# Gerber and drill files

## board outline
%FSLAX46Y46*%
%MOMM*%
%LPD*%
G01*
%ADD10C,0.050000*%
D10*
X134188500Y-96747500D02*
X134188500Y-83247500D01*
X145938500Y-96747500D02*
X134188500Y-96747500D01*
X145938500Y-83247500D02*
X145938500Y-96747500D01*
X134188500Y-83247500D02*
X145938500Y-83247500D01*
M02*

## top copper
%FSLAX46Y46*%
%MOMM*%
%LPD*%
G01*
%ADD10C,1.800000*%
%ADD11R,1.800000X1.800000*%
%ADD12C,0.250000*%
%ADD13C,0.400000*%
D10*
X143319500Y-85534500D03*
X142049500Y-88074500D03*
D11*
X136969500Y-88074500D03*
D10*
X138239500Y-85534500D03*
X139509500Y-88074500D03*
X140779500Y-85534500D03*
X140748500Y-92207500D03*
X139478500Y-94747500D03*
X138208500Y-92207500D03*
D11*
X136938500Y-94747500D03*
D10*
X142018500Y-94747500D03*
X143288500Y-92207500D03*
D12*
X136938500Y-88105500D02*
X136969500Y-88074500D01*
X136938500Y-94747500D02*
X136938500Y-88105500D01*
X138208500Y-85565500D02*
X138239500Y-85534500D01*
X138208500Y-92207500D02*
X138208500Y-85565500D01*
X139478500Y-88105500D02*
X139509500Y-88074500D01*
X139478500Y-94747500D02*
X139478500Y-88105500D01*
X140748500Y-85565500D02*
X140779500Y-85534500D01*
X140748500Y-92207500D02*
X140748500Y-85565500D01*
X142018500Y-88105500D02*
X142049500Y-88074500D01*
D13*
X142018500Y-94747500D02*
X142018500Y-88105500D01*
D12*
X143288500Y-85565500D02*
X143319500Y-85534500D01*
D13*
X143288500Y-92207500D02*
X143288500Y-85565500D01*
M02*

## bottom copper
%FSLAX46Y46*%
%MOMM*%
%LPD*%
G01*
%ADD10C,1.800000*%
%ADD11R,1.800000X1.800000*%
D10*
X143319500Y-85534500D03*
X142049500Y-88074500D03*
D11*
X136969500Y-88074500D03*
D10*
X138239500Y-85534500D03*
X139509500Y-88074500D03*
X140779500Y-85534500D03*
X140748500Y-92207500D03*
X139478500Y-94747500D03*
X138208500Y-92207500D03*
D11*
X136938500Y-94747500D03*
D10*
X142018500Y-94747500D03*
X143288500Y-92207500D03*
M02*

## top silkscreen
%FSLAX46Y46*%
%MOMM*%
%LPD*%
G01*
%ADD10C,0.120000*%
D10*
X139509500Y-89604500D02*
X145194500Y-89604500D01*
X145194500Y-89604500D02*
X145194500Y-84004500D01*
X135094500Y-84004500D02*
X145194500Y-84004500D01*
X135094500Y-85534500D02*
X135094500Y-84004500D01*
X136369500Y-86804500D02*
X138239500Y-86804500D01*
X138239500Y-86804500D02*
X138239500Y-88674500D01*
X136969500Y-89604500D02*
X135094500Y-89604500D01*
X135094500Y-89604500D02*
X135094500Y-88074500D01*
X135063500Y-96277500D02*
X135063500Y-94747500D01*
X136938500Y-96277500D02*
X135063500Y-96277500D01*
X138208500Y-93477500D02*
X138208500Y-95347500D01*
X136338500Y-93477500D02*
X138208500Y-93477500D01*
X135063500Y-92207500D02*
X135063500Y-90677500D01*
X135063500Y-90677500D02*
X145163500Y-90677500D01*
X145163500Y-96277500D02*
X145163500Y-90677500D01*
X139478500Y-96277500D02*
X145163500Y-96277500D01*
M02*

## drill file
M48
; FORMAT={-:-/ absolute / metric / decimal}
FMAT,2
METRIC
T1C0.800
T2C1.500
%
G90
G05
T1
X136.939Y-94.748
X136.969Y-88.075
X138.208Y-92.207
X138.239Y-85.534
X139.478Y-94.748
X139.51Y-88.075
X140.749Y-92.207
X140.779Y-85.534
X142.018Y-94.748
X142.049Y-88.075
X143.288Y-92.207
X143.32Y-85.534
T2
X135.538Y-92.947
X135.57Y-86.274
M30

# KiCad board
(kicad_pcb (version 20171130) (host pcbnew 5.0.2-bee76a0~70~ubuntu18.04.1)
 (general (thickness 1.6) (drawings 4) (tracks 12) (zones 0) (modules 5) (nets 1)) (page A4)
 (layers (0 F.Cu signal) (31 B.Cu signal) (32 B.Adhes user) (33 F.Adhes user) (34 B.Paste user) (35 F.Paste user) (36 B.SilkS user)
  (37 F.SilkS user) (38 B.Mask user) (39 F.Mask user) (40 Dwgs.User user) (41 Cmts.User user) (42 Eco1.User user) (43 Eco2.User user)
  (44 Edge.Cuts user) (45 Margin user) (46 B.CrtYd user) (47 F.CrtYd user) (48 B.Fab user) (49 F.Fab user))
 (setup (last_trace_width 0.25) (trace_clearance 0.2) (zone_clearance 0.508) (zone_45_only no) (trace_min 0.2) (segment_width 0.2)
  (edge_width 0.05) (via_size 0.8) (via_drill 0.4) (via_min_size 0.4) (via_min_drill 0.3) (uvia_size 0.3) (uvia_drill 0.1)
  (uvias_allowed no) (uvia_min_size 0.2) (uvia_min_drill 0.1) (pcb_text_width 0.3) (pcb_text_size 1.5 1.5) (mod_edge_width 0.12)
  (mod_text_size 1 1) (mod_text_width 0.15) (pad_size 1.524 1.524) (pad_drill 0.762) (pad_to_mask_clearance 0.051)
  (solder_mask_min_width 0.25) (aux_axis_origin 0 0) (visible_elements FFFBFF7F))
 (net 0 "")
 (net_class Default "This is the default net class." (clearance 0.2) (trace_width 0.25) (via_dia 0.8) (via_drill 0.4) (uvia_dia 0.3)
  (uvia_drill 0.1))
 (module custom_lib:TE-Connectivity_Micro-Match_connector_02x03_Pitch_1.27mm (layer F.Cu) (at 136.9695 88.0745 90)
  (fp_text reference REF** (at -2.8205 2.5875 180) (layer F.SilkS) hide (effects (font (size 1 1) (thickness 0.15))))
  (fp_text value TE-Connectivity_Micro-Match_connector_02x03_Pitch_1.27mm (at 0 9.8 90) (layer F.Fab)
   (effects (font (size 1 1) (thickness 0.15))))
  (fp_line (start -1.53 2.54) (end -1.53 8.225) (layer F.SilkS) (width 0.12))
  (fp_line (start -1.53 8.225) (end 4.07 8.225) (layer F.SilkS) (width 0.12))
  (fp_line (start 4.07 -1.875) (end 4.07 8.225) (layer F.SilkS) (width 0.12))
  (fp_line (start 2.54 -1.875) (end 4.07 -1.875) (layer F.SilkS) (width 0.12))
  (fp_line (start 1.27 -0.6) (end 1.27 1.27) (layer F.SilkS) (width 0.12))
  (fp_line (start 1.27 1.27) (end -0.6 1.27) (layer F.SilkS) (width 0.12))
  (fp_line (start -1.53 0) (end -1.53 -1.875) (layer F.SilkS) (width 0.12))
  (fp_line (start -1.53 -1.875) (end 0 -1.875) (layer F.SilkS) (width 0.12))
  (pad 6 thru_hole circle (at 2.54 6.35 90) (size 1.8 1.8) (drill 0.8001) (layers *.Cu *.Mask))
  (pad 5 thru_hole circle (at 0 5.08 90) (size 1.8 1.8) (drill 0.8001) (layers *.Cu *.Mask))
  (pad 1 thru_hole rect (at 0 0 90) (size 1.8 1.8) (drill 0.8001) (layers *.Cu *.Mask))
  (pad 2 thru_hole circle (at 2.54 1.27 90) (size 1.8 1.8) (drill 0.8001) (layers *.Cu *.Mask))
  (pad 3 thru_hole circle (at 0 2.54 90) (size 1.8 1.8) (drill 0.8001) (layers *.Cu *.Mask))
  (pad 4 thru_hole circle (at 2.54 3.81 90) (size 1.8 1.8) (drill 0.8001) (layers *.Cu *.Mask))
  (pad "" np_thru_hole circle (at 1.8 -1.4 90) (size 1.5001 1.5001) (drill 1.5001) (layers *.Cu *.Mask)))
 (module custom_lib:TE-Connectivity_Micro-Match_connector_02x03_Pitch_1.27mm (layer F.Cu) (at 136.9385 94.7475 90)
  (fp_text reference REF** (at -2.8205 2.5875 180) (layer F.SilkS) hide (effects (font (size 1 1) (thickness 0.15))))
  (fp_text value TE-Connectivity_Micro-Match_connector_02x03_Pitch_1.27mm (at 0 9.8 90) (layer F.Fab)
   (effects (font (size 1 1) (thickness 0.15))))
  (fp_line (start -1.53 -1.875) (end 0 -1.875) (layer F.SilkS) (width 0.12))
  (fp_line (start -1.53 0) (end -1.53 -1.875) (layer F.SilkS) (width 0.12))
  (fp_line (start 1.27 1.27) (end -0.6 1.27) (layer F.SilkS) (width 0.12))
  (fp_line (start 1.27 -0.6) (end 1.27 1.27) (layer F.SilkS) (width 0.12))
  (fp_line (start 2.54 -1.875) (end 4.07 -1.875) (layer F.SilkS) (width 0.12))
  (fp_line (start 4.07 -1.875) (end 4.07 8.225) (layer F.SilkS) (width 0.12))
  (fp_line (start -1.53 8.225) (end 4.07 8.225) (layer F.SilkS) (width 0.12))
  (fp_line (start -1.53 2.54) (end -1.53 8.225) (layer F.SilkS) (width 0.12))
  (pad "" np_thru_hole circle (at 1.8 -1.4 90) (size 1.5001 1.5001) (drill 1.5001) (layers *.Cu *.Mask))
  (pad 4 thru_hole circle (at 2.54 3.81 90) (size 1.8 1.8) (drill 0.8001) (layers *.Cu *.Mask))
  (pad 3 thru_hole circle (at 0 2.54 90) (size 1.8 1.8) (drill 0.8001) (layers *.Cu *.Mask))
  (pad 2 thru_hole circle (at 2.54 1.27 90) (size 1.8 1.8) (drill 0.8001) (layers *.Cu *.Mask))
  (pad 1 thru_hole rect (at 0 0 90) (size 1.8 1.8) (drill 0.8001) (layers *.Cu *.Mask))
  (pad 5 thru_hole circle (at 0 5.08 90) (size 1.8 1.8) (drill 0.8001) (layers *.Cu *.Mask))
  (pad 6 thru_hole circle (at 2.54 6.35 90) (size 1.8 1.8) (drill 0.8001) (layers *.Cu *.Mask)))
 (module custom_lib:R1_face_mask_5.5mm (layer B.Cu) (at 143.129 90.1065)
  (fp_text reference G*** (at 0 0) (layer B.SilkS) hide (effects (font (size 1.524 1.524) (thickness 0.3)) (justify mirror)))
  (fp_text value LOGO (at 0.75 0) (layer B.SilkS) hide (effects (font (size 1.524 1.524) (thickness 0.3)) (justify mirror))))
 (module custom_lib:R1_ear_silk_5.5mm (layer B.Cu) (at 143.129 90.1065)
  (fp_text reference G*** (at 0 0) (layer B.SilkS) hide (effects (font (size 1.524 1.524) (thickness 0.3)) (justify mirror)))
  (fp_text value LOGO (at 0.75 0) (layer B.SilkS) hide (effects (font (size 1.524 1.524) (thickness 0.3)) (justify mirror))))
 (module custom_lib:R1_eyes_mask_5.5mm (layer B.Cu) (at 143.129 90.1065)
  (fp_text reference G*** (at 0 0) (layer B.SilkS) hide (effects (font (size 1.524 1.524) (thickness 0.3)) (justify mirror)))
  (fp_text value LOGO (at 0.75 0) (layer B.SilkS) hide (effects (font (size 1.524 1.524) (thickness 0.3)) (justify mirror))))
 (gr_line (start 134.1885 96.7475) (end 134.1885 83.2475) (layer Edge.Cuts) (width 0.05))
 (gr_line (start 145.9385 96.7475) (end 134.1885 96.7475) (layer Edge.Cuts) (width 0.05))
 (gr_line (start 145.9385 83.2475) (end 145.9385 96.7475) (layer Edge.Cuts) (width 0.05))
 (gr_line (start 134.1885 83.2475) (end 145.9385 83.2475) (layer Edge.Cuts) (width 0.05))
 (segment (start 136.9385 88.1055) (end 136.9695 88.0745) (width 0.25) (layer F.Cu) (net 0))
 (segment (start 136.9385 94.7475) (end 136.9385 88.1055) (width 0.25) (layer F.Cu) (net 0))
 (segment (start 138.2085 85.5655) (end 138.2395 85.5345) (width 0.25) (layer F.Cu) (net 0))
 (segment (start 138.2085 92.2075) (end 138.2085 85.5655) (width 0.25) (layer F.Cu) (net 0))
 (segment (start 139.4785 88.1055) (end 139.5095 88.0745) (width 0.25) (layer F.Cu) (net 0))
 (segment (start 139.4785 94.7475) (end 139.4785 88.1055) (width 0.25) (layer F.Cu) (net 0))
 (segment (start 140.7485 85.5655) (end 140.7795 85.5345) (width 0.25) (layer F.Cu) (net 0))
 (segment (start 140.7485 92.2075) (end 140.7485 85.5655) (width 0.25) (layer F.Cu) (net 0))
 (segment (start 142.0185 88.1055) (end 142.0495 88.0745) (width 0.25) (layer F.Cu) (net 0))
 (segment (start 142.0185 94.7475) (end 142.0185 88.1055) (width 0.4) (layer F.Cu) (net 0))
 (segment (start 143.2885 85.5655) (end 143.3195 85.5345) (width 0.25) (layer F.Cu) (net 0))
 (segment (start 143.2885 92.2075) (end 143.2885 85.5655) (width 0.4) (layer F.Cu) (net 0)))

